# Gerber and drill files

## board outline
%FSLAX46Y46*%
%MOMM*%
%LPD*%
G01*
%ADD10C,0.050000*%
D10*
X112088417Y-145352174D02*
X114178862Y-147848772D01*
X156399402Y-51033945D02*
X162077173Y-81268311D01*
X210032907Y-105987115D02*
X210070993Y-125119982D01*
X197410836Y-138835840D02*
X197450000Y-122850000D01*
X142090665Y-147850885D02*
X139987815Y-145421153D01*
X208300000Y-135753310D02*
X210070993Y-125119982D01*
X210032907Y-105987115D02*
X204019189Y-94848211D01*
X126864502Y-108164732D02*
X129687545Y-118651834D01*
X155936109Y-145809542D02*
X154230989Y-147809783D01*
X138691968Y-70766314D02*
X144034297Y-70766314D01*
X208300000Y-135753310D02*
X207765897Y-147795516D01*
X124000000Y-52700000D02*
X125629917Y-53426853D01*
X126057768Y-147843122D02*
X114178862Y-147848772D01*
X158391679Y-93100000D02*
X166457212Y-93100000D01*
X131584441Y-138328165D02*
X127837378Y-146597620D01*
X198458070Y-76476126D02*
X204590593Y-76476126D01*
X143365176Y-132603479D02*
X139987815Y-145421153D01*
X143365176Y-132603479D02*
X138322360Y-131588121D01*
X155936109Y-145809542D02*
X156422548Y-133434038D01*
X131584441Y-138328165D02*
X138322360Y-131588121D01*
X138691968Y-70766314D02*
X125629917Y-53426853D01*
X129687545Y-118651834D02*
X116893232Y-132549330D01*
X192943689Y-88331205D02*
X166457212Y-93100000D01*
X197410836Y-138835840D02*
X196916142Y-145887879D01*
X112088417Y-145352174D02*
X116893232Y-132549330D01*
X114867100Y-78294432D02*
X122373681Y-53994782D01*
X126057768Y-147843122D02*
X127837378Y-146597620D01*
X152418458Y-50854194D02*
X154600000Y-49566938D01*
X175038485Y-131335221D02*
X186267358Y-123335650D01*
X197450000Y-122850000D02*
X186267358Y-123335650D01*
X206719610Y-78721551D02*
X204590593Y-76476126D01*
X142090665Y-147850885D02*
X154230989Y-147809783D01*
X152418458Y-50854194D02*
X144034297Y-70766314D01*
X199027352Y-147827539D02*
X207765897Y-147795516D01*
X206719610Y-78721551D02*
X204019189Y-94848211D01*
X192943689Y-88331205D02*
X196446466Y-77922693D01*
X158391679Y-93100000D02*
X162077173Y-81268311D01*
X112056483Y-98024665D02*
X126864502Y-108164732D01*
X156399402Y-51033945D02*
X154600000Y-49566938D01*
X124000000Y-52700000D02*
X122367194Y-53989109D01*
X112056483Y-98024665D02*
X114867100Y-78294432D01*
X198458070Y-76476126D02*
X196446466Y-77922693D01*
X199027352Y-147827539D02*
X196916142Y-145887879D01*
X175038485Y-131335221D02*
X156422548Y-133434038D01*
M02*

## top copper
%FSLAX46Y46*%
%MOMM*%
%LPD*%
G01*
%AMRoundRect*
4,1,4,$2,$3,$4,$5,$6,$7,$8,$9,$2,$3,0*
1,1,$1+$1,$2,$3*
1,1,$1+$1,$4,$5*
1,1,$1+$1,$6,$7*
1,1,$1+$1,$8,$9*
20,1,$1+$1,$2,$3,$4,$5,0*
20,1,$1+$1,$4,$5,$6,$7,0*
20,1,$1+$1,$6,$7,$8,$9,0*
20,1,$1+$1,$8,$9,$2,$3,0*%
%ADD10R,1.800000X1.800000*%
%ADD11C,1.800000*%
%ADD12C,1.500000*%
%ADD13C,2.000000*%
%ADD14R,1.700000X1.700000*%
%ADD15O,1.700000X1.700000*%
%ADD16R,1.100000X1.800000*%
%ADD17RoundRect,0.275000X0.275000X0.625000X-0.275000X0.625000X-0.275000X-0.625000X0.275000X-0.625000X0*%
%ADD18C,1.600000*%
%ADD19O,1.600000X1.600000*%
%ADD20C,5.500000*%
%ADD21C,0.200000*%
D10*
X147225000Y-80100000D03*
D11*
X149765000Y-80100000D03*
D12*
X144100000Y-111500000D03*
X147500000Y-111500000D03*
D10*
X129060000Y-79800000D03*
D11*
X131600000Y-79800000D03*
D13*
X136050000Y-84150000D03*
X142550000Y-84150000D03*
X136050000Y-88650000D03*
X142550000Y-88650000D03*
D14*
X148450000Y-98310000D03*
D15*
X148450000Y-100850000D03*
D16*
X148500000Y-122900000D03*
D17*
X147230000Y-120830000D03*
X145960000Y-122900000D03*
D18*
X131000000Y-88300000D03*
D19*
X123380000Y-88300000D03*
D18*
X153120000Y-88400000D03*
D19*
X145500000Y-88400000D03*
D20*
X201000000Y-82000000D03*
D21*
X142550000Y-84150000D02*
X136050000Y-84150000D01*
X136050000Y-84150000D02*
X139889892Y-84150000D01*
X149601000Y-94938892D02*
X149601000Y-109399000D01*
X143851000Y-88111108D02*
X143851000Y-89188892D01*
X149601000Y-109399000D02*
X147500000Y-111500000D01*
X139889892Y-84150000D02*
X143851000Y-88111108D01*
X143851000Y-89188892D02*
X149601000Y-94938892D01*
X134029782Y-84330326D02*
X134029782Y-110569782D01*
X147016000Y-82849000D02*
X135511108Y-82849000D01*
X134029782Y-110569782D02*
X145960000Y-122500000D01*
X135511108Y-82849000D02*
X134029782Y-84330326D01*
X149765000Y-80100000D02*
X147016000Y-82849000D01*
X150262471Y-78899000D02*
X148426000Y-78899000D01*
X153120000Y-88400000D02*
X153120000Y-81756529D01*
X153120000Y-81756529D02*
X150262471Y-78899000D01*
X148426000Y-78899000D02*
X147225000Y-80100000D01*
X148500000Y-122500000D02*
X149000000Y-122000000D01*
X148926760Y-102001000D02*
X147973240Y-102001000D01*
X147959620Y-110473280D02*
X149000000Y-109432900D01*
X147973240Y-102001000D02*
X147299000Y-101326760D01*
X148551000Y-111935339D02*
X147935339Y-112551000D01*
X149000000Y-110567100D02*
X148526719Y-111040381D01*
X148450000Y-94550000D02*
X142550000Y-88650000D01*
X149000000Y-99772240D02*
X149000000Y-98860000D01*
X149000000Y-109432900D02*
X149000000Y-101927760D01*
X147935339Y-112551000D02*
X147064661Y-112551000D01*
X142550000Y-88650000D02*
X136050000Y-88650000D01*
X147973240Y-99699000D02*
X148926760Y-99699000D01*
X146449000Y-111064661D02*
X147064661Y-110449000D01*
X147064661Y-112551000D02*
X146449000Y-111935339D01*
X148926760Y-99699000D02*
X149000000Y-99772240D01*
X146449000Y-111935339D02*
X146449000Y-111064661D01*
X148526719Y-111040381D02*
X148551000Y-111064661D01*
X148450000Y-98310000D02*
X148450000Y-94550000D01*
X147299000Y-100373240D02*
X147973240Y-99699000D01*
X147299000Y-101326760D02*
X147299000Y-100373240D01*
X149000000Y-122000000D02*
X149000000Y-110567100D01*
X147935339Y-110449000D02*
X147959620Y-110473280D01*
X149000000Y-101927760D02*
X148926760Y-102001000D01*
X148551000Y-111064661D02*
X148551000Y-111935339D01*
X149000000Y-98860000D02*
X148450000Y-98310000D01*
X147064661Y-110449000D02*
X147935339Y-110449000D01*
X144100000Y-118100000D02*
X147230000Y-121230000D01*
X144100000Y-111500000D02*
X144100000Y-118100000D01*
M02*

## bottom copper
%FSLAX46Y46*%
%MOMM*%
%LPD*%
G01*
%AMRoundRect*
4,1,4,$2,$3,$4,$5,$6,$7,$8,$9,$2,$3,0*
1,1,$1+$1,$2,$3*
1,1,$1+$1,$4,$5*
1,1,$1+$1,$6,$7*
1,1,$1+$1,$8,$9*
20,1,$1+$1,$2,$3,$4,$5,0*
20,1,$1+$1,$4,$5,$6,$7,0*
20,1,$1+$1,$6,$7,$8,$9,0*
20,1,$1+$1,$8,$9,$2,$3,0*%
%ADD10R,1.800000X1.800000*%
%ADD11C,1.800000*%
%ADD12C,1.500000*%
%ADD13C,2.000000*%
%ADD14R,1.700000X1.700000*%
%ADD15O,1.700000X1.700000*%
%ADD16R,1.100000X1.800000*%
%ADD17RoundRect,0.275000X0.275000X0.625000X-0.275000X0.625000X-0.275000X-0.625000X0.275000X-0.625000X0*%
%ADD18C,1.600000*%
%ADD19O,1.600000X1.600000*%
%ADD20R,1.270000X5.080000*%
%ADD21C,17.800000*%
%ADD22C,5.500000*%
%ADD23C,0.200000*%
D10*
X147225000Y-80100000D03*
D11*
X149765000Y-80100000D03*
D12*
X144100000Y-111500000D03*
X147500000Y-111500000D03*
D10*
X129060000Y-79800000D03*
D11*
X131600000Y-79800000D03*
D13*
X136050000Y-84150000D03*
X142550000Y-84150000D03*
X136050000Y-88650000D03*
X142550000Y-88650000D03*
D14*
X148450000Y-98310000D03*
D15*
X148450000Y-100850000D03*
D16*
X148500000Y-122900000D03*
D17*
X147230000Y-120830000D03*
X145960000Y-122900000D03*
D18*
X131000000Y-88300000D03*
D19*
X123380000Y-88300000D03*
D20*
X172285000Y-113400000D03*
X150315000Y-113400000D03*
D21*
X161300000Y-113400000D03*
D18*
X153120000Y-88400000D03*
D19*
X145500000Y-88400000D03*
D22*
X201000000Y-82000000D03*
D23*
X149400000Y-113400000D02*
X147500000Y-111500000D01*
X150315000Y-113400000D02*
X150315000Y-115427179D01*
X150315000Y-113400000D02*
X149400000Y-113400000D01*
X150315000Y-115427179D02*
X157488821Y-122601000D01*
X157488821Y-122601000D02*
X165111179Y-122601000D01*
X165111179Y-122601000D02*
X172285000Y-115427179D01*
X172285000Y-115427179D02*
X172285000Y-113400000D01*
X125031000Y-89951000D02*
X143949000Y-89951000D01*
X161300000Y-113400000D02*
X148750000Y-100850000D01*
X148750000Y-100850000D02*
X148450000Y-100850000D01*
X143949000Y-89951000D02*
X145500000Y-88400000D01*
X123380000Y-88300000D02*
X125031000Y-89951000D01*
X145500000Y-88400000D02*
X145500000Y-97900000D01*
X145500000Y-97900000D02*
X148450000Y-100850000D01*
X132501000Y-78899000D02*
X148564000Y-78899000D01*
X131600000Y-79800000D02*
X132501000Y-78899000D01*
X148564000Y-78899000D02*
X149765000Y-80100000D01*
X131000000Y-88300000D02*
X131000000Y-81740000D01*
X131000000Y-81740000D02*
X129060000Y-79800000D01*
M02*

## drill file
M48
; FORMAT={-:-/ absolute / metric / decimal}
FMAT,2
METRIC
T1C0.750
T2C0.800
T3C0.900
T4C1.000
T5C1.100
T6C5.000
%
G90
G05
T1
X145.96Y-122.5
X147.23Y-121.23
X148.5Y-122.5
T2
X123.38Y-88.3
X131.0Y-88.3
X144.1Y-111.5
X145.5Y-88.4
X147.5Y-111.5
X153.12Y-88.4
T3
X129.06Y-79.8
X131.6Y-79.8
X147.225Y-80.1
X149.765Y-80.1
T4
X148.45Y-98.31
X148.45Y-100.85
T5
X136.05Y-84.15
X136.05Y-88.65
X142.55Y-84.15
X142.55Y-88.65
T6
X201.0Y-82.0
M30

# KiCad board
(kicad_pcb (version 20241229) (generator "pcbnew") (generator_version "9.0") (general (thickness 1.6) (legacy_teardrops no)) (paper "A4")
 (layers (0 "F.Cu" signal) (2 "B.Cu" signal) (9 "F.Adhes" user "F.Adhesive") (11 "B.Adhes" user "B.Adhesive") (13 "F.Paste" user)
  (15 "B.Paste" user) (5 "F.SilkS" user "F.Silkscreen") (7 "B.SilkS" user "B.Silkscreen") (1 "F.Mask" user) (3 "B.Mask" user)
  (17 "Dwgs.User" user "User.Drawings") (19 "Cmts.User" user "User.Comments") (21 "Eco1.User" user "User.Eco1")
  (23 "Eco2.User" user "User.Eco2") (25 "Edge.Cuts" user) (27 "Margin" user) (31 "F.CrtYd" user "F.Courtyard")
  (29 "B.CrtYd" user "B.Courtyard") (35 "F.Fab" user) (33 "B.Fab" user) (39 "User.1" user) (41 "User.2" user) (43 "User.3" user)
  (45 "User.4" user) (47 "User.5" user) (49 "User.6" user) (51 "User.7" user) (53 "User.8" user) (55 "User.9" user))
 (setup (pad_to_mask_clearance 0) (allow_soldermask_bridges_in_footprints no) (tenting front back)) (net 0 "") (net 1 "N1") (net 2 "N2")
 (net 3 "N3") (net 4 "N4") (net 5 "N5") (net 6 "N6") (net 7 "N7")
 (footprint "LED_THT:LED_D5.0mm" (layer "F.Cu") (at 147.225 80.1)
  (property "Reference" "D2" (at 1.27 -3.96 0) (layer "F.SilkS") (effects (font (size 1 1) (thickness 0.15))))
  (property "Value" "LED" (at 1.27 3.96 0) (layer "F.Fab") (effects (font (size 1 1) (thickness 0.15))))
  (pad "1" thru_hole rect (at 0 0) (size 1.8 1.8) (drill 0.9) (layers "*.Cu" "*.Mask") (remove_unused_layers no) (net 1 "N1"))
  (pad "2" thru_hole circle (at 2.54 0) (size 1.8 1.8) (drill 0.9) (layers "*.Cu" "*.Mask") (remove_unused_layers no) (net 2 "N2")))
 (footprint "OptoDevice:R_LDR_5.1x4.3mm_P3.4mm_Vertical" (layer "F.Cu") (at 144.1 111.5)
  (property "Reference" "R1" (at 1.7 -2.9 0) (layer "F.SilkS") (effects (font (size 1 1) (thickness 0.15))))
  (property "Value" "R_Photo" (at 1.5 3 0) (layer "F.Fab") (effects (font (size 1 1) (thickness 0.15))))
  (pad "1" thru_hole circle (at 0 0) (size 1.5 1.5) (drill 0.8) (layers "*.Cu" "*.Mask") (remove_unused_layers no) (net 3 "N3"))
  (pad "2" thru_hole circle (at 3.4 0) (size 1.5 1.5) (drill 0.8) (layers "*.Cu" "*.Mask") (remove_unused_layers no) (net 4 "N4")))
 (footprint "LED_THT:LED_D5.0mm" (layer "F.Cu") (at 129.06 79.8)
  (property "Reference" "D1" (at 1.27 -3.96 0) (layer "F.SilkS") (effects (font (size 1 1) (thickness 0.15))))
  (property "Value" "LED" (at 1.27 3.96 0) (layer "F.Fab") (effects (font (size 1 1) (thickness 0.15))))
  (pad "1" thru_hole rect (at 0 0) (size 1.8 1.8) (drill 0.9) (layers "*.Cu" "*.Mask") (remove_unused_layers no) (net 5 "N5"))
  (pad "2" thru_hole circle (at 2.54 0) (size 1.8 1.8) (drill 0.9) (layers "*.Cu" "*.Mask") (remove_unused_layers no) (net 2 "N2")))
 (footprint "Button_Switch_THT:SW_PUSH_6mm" (layer "F.Cu") (at 136.05 84.15)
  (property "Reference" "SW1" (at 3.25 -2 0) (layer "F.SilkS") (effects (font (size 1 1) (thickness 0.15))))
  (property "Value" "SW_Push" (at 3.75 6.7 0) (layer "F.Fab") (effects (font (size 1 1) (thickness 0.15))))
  (pad "1" thru_hole circle (at 0 0 90) (size 2 2) (drill 1.1) (layers "*.Cu" "*.Mask") (remove_unused_layers no) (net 4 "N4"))
  (pad "1" thru_hole circle (at 6.5 0 90) (size 2 2) (drill 1.1) (layers "*.Cu" "*.Mask") (remove_unused_layers no) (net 4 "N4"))
  (pad "2" thru_hole circle (at 0 4.5 90) (size 2 2) (drill 1.1) (layers "*.Cu" "*.Mask") (remove_unused_layers no) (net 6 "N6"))
  (pad "2" thru_hole circle (at 6.5 4.5 90) (size 2 2) (drill 1.1) (layers "*.Cu" "*.Mask") (remove_unused_layers no) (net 6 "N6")))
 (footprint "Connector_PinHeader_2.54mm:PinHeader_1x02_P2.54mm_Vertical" (layer "B.Cu") (at 148.45 98.31 180)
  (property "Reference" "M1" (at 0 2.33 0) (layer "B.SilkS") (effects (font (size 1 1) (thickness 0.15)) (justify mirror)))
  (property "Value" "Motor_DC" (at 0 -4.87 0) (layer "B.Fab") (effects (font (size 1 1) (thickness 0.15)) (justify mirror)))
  (pad "1" thru_hole rect (at 0 0 180) (size 1.7 1.7) (drill 1) (layers "*.Cu" "*.Mask") (remove_unused_layers no) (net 6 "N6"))
  (pad "2" thru_hole oval (at 0 -2.54 180) (size 1.7 1.7) (drill 1) (layers "*.Cu" "*.Mask") (remove_unused_layers no) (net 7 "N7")))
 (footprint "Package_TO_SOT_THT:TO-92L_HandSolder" (layer "B.Cu") (at 148.5 122.5 180)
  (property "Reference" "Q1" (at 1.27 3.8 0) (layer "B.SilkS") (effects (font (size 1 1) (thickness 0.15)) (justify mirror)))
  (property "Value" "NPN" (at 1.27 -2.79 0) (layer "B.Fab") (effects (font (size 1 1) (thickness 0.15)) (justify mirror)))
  (pad "1" thru_hole rect (at 0 0 180) (size 1.1 1.8) (drill 0.75 (offset 0 -0.4)) (layers "*.Cu" "*.Mask") (remove_unused_layers no)
   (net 6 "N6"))
  (pad "2" thru_hole roundrect (at 1.27 1.27 180) (size 1.1 1.8) (drill 0.75 (offset 0 0.4)) (layers "*.Cu" "*.Mask")
   (remove_unused_layers no) (roundrect_rratio 0.25) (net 3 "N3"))
  (pad "3" thru_hole roundrect (at 2.54 0 180) (size 1.1 1.8) (drill 0.75 (offset 0 -0.4)) (layers "*.Cu" "*.Mask")
   (remove_unused_layers no) (roundrect_rratio 0.25) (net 2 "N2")))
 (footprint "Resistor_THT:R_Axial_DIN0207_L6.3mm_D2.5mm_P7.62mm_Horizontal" (layer "B.Cu") (at 131 88.3 180)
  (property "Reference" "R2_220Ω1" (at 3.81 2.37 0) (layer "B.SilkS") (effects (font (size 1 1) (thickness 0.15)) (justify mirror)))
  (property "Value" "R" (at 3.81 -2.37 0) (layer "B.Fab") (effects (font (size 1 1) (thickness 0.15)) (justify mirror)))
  (pad "1" thru_hole circle (at 0 0 180) (size 1.6 1.6) (drill 0.8) (layers "*.Cu" "*.Mask") (remove_unused_layers no) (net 5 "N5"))
  (pad "2" thru_hole oval (at 7.62 0 180) (size 1.6 1.6) (drill 0.8) (layers "*.Cu" "*.Mask") (remove_unused_layers no) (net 7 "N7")))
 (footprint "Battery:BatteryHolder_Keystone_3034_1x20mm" (layer "B.Cu") (at 161.3 113.4 180)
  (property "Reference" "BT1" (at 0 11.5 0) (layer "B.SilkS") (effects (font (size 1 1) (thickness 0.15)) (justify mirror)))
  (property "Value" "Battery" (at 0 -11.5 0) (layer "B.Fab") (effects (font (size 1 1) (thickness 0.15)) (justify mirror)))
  (pad "1" smd rect (at -10.985 0 180) (size 1.27 5.08) (layers "B.Cu" "B.Mask" "B.Paste") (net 4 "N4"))
  (pad "1" smd rect (at 10.985 0 180) (size 1.27 5.08) (layers "B.Cu" "B.Mask" "B.Paste") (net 4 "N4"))
  (pad "2" smd circle (at 0 0 180) (size 17.8 17.8) (layers "B.Cu" "B.Mask") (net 7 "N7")))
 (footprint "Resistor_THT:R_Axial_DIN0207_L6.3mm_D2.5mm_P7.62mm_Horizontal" (layer "B.Cu") (at 153.12 88.4 180)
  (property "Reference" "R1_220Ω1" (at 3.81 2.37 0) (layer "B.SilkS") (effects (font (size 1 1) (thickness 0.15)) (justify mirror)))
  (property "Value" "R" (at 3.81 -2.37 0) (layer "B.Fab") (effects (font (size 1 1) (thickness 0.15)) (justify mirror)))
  (pad "1" thru_hole circle (at 0 0 180) (size 1.6 1.6) (drill 0.8) (layers "*.Cu" "*.Mask") (remove_unused_layers no) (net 1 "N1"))
  (pad "2" thru_hole oval (at 7.62 0 180) (size 1.6 1.6) (drill 0.8) (layers "*.Cu" "*.Mask") (remove_unused_layers no) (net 7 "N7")))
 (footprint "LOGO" (layer "B.Cu") (at 183 113.5 180)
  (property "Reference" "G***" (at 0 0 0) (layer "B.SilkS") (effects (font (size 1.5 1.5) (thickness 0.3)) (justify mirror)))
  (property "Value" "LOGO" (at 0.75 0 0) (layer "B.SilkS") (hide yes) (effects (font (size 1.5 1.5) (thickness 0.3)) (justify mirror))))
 (gr_line (start 112.088417 145.352174) (end 114.178862 147.848772) (stroke (width 0.05) (type default)) (layer "Edge.Cuts"))
 (gr_line (start 156.399402 51.033945) (end 162.077173 81.268311) (stroke (width 0.05) (type default)) (layer "Edge.Cuts"))
 (gr_line (start 210.032907 105.987115) (end 210.070993 125.119982) (stroke (width 0.05) (type default)) (layer "Edge.Cuts"))
 (gr_line (start 197.410836 138.83584) (end 197.45 122.85) (stroke (width 0.05) (type default)) (layer "Edge.Cuts"))
 (gr_line (start 142.090665 147.850885) (end 139.987815 145.421153) (stroke (width 0.05) (type default)) (layer "Edge.Cuts"))
 (gr_line (start 208.3 135.75331) (end 210.070993 125.119982) (stroke (width 0.05) (type default)) (layer "Edge.Cuts"))
 (gr_line (start 210.032907 105.987115) (end 204.019189 94.848211) (stroke (width 0.05) (type default)) (layer "Edge.Cuts"))
 (gr_line (start 126.864502 108.164732) (end 129.687545 118.651834) (stroke (width 0.05) (type default)) (layer "Edge.Cuts"))
 (gr_line (start 155.936109 145.809542) (end 154.230989 147.809783) (stroke (width 0.05) (type default)) (layer "Edge.Cuts"))
 (gr_line (start 138.691968 70.766314) (end 144.034297 70.766314) (stroke (width 0.05) (type default)) (layer "Edge.Cuts"))
 (gr_line (start 208.3 135.75331) (end 207.765897 147.795516) (stroke (width 0.05) (type default)) (layer "Edge.Cuts"))
 (gr_line (start 124 52.7) (end 125.629917 53.426853) (stroke (width 0.05) (type default)) (layer "Edge.Cuts"))
 (gr_line (start 126.057768 147.843122) (end 114.178862 147.848772) (stroke (width 0.05) (type default)) (layer "Edge.Cuts"))
 (gr_line (start 158.391679 93.1) (end 166.457212 93.1) (stroke (width 0.05) (type default)) (layer "Edge.Cuts"))
 (gr_line (start 131.584441 138.328165) (end 127.837378 146.59762) (stroke (width 0.05) (type default)) (layer "Edge.Cuts"))
 (gr_line (start 198.45807 76.476126) (end 204.590593 76.476126) (stroke (width 0.05) (type default)) (layer "Edge.Cuts"))
 (gr_line (start 143.365176 132.603479) (end 139.987815 145.421153) (stroke (width 0.05) (type default)) (layer "Edge.Cuts"))
 (gr_line (start 143.365176 132.603479) (end 138.32236 131.588121) (stroke (width 0.05) (type default)) (layer "Edge.Cuts"))
 (gr_line (start 155.936109 145.809542) (end 156.422548 133.434038) (stroke (width 0.05) (type default)) (layer "Edge.Cuts"))
 (gr_line (start 131.584441 138.328165) (end 138.32236 131.588121) (stroke (width 0.05) (type default)) (layer "Edge.Cuts"))
 (gr_line (start 138.691968 70.766314) (end 125.629917 53.426853) (stroke (width 0.05) (type default)) (layer "Edge.Cuts"))
 (gr_line (start 129.687545 118.651834) (end 116.893232 132.54933) (stroke (width 0.05) (type default)) (layer "Edge.Cuts"))
 (gr_line (start 192.943689 88.331205) (end 166.457212 93.1) (stroke (width 0.05) (type default)) (layer "Edge.Cuts"))
 (gr_line (start 197.410836 138.83584) (end 196.916142 145.887879) (stroke (width 0.05) (type default)) (layer "Edge.Cuts"))
 (gr_line (start 112.088417 145.352174) (end 116.893232 132.54933) (stroke (width 0.05) (type default)) (layer "Edge.Cuts"))
 (gr_line (start 114.8671 78.294432) (end 122.373681 53.994782) (stroke (width 0.05) (type default)) (layer "Edge.Cuts"))
 (gr_line (start 126.057768 147.843122) (end 127.837378 146.59762) (stroke (width 0.05) (type default)) (layer "Edge.Cuts"))
 (gr_line (start 152.418458 50.854194) (end 154.6 49.566938) (stroke (width 0.05) (type default)) (layer "Edge.Cuts"))
 (gr_line (start 175.038485 131.335221) (end 186.267358 123.33565) (stroke (width 0.05) (type default)) (layer "Edge.Cuts"))
 (gr_line (start 197.45 122.85) (end 186.267358 123.33565) (stroke (width 0.05) (type default)) (layer "Edge.Cuts"))
 (gr_line (start 206.71961 78.721551) (end 204.590593 76.476126) (stroke (width 0.05) (type default)) (layer "Edge.Cuts"))
 (gr_line (start 142.090665 147.850885) (end 154.230989 147.809783) (stroke (width 0.05) (type default)) (layer "Edge.Cuts"))
 (gr_line (start 152.418458 50.854194) (end 144.034297 70.766314) (stroke (width 0.05) (type default)) (layer "Edge.Cuts"))
 (gr_line (start 199.027352 147.827539) (end 207.765897 147.795516) (stroke (width 0.05) (type default)) (layer "Edge.Cuts"))
 (gr_line (start 206.71961 78.721551) (end 204.019189 94.848211) (stroke (width 0.05) (type default)) (layer "Edge.Cuts"))
 (gr_line (start 192.943689 88.331205) (end 196.446466 77.922693) (stroke (width 0.05) (type default)) (layer "Edge.Cuts"))
 (gr_line (start 158.391679 93.1) (end 162.077173 81.268311) (stroke (width 0.05) (type default)) (layer "Edge.Cuts"))
 (gr_line (start 112.056483 98.024665) (end 126.864502 108.164732) (stroke (width 0.05) (type default)) (layer "Edge.Cuts"))
 (gr_line (start 156.399402 51.033945) (end 154.6 49.566938) (stroke (width 0.05) (type default)) (layer "Edge.Cuts"))
 (gr_line (start 124 52.7) (end 122.367194 53.989109) (stroke (width 0.05) (type default)) (layer "Edge.Cuts"))
 (gr_line (start 112.056483 98.024665) (end 114.8671 78.294432) (stroke (width 0.05) (type default)) (layer "Edge.Cuts"))
 (gr_line (start 198.45807 76.476126) (end 196.446466 77.922693) (stroke (width 0.05) (type default)) (layer "Edge.Cuts"))
 (gr_line (start 199.027352 147.827539) (end 196.916142 145.887879) (stroke (width 0.05) (type default)) (layer "Edge.Cuts"))
 (gr_line (start 175.038485 131.335221) (end 156.422548 133.434038) (stroke (width 0.05) (type default)) (layer "Edge.Cuts"))
 (via (at 201 82) (size 5.5) (drill 5) (layers "F.Cu" "B.Cu") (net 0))
 (segment (start 142.55 84.15) (end 136.05 84.15) (width 0.2) (layer "F.Cu") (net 4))
 (segment (start 136.05 84.15) (end 139.889892 84.15) (width 0.2) (layer "F.Cu") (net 4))
 (segment (start 149.601 94.938892) (end 149.601 109.399) (width 0.2) (layer "F.Cu") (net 4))
 (segment (start 143.851 88.111108) (end 143.851 89.188892) (width 0.2) (layer "F.Cu") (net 4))
 (segment (start 149.601 109.399) (end 147.5 111.5) (width 0.2) (layer "F.Cu") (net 4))
 (segment (start 139.889892 84.15) (end 143.851 88.111108) (width 0.2) (layer "F.Cu") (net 4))
 (segment (start 143.851 89.188892) (end 149.601 94.938892) (width 0.2) (layer "F.Cu") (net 4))
 (segment (start 149.4 113.4) (end 147.5 111.5) (width 0.2) (layer "B.Cu") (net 4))
 (segment (start 150.315 113.4) (end 150.315 115.427179) (width 0.2) (layer "B.Cu") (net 4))
 (segment (start 150.315 113.4) (end 149.4 113.4) (width 0.2) (layer "B.Cu") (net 4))
 (segment (start 150.315 115.427179) (end 157.488821 122.601) (width 0.2) (layer "B.Cu") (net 4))
 (segment (start 157.488821 122.601) (end 165.111179 122.601) (width 0.2) (layer "B.Cu") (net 4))
 (segment (start 165.111179 122.601) (end 172.285 115.427179) (width 0.2) (layer "B.Cu") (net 4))
 (segment (start 172.285 115.427179) (end 172.285 113.4) (width 0.2) (layer "B.Cu") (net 4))
 (segment (start 125.031 89.951) (end 143.949 89.951) (width 0.2) (layer "B.Cu") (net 7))
 (segment (start 161.3 113.4) (end 148.75 100.85) (width 0.2) (layer "B.Cu") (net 7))
 (segment (start 148.75 100.85) (end 148.45 100.85) (width 0.2) (layer "B.Cu") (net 7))
 (segment (start 143.949 89.951) (end 145.5 88.4) (width 0.2) (layer "B.Cu") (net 7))
 (segment (start 123.38 88.3) (end 125.031 89.951) (width 0.2) (layer "B.Cu") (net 7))
 (segment (start 145.5 88.4) (end 145.5 97.9) (width 0.2) (layer "B.Cu") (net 7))
 (segment (start 145.5 97.9) (end 148.45 100.85) (width 0.2) (layer "B.Cu") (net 7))
 (segment (start 134.029782 84.330326) (end 134.029782 110.569782) (width 0.2) (layer "F.Cu") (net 2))
 (segment (start 147.016 82.849) (end 135.511108 82.849) (width 0.2) (layer "F.Cu") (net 2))
 (segment (start 134.029782 110.569782) (end 145.96 122.5) (width 0.2) (layer "F.Cu") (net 2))
 (segment (start 135.511108 82.849) (end 134.029782 84.330326) (width 0.2) (layer "F.Cu") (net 2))
 (segment (start 149.765 80.1) (end 147.016 82.849) (width 0.2) (layer "F.Cu") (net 2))
 (segment (start 132.501 78.899) (end 148.564 78.899) (width 0.2) (layer "B.Cu") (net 2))
 (segment (start 131.6 79.8) (end 132.501 78.899) (width 0.2) (layer "B.Cu") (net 2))
 (segment (start 148.564 78.899) (end 149.765 80.1) (width 0.2) (layer "B.Cu") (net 2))
 (segment (start 131 88.3) (end 131 81.74) (width 0.2) (layer "B.Cu") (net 5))
 (segment (start 131 81.74) (end 129.06 79.8) (width 0.2) (layer "B.Cu") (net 5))
 (segment (start 150.262471 78.899) (end 148.426 78.899) (width 0.2) (layer "F.Cu") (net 1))
 (segment (start 153.12 88.4) (end 153.12 81.756529) (width 0.2) (layer "F.Cu") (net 1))
 (segment (start 153.12 81.756529) (end 150.262471 78.899) (width 0.2) (layer "F.Cu") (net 1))
 (segment (start 148.426 78.899) (end 147.225 80.1) (width 0.2) (layer "F.Cu") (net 1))
 (segment (start 148.5 122.5) (end 149 122) (width 0.2) (layer "F.Cu") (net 6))
 (segment (start 148.92676 102.001) (end 147.97324 102.001) (width 0.2) (layer "F.Cu") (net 6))
 (segment (start 147.95962 110.47328) (end 149 109.4329) (width 0.2) (layer "F.Cu") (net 6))
 (segment (start 147.97324 102.001) (end 147.299 101.32676) (width 0.2) (layer "F.Cu") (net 6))
 (segment (start 148.551 111.935339) (end 147.935339 112.551) (width 0.2) (layer "F.Cu") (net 6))
 (segment (start 149 110.5671) (end 148.526719 111.040381) (width 0.2) (layer "F.Cu") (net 6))
 (segment (start 148.45 94.55) (end 142.55 88.65) (width 0.2) (layer "F.Cu") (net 6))
 (segment (start 149 99.77224) (end 149 98.86) (width 0.2) (layer "F.Cu") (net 6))
 (segment (start 149 109.4329) (end 149 101.92776) (width 0.2) (layer "F.Cu") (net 6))
 (segment (start 147.935339 112.551) (end 147.064661 112.551) (width 0.2) (layer "F.Cu") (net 6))
 (segment (start 142.55 88.65) (end 136.05 88.65) (width 0.2) (layer "F.Cu") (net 6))
 (segment (start 147.97324 99.699) (end 148.92676 99.699) (width 0.2) (layer "F.Cu") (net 6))
 (segment (start 146.449 111.064661) (end 147.064661 110.449) (width 0.2) (layer "F.Cu") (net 6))
 (segment (start 147.064661 112.551) (end 146.449 111.935339) (width 0.2) (layer "F.Cu") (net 6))
 (segment (start 148.92676 99.699) (end 149 99.77224) (width 0.2) (layer "F.Cu") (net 6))
 (segment (start 146.449 111.935339) (end 146.449 111.064661) (width 0.2) (layer "F.Cu") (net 6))
 (segment (start 148.526719 111.040381) (end 148.551 111.064661) (width 0.2) (layer "F.Cu") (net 6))
 (segment (start 148.45 98.31) (end 148.45 94.55) (width 0.2) (layer "F.Cu") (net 6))
 (segment (start 147.299 100.37324) (end 147.97324 99.699) (width 0.2) (layer "F.Cu") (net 6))
 (segment (start 147.299 101.32676) (end 147.299 100.37324) (width 0.2) (layer "F.Cu") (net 6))
 (segment (start 149 122) (end 149 110.5671) (width 0.2) (layer "F.Cu") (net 6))
 (segment (start 147.935339 110.449) (end 147.95962 110.47328) (width 0.2) (layer "F.Cu") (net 6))
 (segment (start 149 101.92776) (end 148.92676 102.001) (width 0.2) (layer "F.Cu") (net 6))
 (segment (start 148.551 111.064661) (end 148.551 111.935339) (width 0.2) (layer "F.Cu") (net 6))
 (segment (start 149 98.86) (end 148.45 98.31) (width 0.2) (layer "F.Cu") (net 6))
 (segment (start 147.064661 110.449) (end 147.935339 110.449) (width 0.2) (layer "F.Cu") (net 6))
 (segment (start 144.1 118.1) (end 147.23 121.23) (width 0.2) (layer "F.Cu") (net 3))
 (segment (start 144.1 111.5) (end 144.1 118.1) (width 0.2) (layer "F.Cu") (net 3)))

